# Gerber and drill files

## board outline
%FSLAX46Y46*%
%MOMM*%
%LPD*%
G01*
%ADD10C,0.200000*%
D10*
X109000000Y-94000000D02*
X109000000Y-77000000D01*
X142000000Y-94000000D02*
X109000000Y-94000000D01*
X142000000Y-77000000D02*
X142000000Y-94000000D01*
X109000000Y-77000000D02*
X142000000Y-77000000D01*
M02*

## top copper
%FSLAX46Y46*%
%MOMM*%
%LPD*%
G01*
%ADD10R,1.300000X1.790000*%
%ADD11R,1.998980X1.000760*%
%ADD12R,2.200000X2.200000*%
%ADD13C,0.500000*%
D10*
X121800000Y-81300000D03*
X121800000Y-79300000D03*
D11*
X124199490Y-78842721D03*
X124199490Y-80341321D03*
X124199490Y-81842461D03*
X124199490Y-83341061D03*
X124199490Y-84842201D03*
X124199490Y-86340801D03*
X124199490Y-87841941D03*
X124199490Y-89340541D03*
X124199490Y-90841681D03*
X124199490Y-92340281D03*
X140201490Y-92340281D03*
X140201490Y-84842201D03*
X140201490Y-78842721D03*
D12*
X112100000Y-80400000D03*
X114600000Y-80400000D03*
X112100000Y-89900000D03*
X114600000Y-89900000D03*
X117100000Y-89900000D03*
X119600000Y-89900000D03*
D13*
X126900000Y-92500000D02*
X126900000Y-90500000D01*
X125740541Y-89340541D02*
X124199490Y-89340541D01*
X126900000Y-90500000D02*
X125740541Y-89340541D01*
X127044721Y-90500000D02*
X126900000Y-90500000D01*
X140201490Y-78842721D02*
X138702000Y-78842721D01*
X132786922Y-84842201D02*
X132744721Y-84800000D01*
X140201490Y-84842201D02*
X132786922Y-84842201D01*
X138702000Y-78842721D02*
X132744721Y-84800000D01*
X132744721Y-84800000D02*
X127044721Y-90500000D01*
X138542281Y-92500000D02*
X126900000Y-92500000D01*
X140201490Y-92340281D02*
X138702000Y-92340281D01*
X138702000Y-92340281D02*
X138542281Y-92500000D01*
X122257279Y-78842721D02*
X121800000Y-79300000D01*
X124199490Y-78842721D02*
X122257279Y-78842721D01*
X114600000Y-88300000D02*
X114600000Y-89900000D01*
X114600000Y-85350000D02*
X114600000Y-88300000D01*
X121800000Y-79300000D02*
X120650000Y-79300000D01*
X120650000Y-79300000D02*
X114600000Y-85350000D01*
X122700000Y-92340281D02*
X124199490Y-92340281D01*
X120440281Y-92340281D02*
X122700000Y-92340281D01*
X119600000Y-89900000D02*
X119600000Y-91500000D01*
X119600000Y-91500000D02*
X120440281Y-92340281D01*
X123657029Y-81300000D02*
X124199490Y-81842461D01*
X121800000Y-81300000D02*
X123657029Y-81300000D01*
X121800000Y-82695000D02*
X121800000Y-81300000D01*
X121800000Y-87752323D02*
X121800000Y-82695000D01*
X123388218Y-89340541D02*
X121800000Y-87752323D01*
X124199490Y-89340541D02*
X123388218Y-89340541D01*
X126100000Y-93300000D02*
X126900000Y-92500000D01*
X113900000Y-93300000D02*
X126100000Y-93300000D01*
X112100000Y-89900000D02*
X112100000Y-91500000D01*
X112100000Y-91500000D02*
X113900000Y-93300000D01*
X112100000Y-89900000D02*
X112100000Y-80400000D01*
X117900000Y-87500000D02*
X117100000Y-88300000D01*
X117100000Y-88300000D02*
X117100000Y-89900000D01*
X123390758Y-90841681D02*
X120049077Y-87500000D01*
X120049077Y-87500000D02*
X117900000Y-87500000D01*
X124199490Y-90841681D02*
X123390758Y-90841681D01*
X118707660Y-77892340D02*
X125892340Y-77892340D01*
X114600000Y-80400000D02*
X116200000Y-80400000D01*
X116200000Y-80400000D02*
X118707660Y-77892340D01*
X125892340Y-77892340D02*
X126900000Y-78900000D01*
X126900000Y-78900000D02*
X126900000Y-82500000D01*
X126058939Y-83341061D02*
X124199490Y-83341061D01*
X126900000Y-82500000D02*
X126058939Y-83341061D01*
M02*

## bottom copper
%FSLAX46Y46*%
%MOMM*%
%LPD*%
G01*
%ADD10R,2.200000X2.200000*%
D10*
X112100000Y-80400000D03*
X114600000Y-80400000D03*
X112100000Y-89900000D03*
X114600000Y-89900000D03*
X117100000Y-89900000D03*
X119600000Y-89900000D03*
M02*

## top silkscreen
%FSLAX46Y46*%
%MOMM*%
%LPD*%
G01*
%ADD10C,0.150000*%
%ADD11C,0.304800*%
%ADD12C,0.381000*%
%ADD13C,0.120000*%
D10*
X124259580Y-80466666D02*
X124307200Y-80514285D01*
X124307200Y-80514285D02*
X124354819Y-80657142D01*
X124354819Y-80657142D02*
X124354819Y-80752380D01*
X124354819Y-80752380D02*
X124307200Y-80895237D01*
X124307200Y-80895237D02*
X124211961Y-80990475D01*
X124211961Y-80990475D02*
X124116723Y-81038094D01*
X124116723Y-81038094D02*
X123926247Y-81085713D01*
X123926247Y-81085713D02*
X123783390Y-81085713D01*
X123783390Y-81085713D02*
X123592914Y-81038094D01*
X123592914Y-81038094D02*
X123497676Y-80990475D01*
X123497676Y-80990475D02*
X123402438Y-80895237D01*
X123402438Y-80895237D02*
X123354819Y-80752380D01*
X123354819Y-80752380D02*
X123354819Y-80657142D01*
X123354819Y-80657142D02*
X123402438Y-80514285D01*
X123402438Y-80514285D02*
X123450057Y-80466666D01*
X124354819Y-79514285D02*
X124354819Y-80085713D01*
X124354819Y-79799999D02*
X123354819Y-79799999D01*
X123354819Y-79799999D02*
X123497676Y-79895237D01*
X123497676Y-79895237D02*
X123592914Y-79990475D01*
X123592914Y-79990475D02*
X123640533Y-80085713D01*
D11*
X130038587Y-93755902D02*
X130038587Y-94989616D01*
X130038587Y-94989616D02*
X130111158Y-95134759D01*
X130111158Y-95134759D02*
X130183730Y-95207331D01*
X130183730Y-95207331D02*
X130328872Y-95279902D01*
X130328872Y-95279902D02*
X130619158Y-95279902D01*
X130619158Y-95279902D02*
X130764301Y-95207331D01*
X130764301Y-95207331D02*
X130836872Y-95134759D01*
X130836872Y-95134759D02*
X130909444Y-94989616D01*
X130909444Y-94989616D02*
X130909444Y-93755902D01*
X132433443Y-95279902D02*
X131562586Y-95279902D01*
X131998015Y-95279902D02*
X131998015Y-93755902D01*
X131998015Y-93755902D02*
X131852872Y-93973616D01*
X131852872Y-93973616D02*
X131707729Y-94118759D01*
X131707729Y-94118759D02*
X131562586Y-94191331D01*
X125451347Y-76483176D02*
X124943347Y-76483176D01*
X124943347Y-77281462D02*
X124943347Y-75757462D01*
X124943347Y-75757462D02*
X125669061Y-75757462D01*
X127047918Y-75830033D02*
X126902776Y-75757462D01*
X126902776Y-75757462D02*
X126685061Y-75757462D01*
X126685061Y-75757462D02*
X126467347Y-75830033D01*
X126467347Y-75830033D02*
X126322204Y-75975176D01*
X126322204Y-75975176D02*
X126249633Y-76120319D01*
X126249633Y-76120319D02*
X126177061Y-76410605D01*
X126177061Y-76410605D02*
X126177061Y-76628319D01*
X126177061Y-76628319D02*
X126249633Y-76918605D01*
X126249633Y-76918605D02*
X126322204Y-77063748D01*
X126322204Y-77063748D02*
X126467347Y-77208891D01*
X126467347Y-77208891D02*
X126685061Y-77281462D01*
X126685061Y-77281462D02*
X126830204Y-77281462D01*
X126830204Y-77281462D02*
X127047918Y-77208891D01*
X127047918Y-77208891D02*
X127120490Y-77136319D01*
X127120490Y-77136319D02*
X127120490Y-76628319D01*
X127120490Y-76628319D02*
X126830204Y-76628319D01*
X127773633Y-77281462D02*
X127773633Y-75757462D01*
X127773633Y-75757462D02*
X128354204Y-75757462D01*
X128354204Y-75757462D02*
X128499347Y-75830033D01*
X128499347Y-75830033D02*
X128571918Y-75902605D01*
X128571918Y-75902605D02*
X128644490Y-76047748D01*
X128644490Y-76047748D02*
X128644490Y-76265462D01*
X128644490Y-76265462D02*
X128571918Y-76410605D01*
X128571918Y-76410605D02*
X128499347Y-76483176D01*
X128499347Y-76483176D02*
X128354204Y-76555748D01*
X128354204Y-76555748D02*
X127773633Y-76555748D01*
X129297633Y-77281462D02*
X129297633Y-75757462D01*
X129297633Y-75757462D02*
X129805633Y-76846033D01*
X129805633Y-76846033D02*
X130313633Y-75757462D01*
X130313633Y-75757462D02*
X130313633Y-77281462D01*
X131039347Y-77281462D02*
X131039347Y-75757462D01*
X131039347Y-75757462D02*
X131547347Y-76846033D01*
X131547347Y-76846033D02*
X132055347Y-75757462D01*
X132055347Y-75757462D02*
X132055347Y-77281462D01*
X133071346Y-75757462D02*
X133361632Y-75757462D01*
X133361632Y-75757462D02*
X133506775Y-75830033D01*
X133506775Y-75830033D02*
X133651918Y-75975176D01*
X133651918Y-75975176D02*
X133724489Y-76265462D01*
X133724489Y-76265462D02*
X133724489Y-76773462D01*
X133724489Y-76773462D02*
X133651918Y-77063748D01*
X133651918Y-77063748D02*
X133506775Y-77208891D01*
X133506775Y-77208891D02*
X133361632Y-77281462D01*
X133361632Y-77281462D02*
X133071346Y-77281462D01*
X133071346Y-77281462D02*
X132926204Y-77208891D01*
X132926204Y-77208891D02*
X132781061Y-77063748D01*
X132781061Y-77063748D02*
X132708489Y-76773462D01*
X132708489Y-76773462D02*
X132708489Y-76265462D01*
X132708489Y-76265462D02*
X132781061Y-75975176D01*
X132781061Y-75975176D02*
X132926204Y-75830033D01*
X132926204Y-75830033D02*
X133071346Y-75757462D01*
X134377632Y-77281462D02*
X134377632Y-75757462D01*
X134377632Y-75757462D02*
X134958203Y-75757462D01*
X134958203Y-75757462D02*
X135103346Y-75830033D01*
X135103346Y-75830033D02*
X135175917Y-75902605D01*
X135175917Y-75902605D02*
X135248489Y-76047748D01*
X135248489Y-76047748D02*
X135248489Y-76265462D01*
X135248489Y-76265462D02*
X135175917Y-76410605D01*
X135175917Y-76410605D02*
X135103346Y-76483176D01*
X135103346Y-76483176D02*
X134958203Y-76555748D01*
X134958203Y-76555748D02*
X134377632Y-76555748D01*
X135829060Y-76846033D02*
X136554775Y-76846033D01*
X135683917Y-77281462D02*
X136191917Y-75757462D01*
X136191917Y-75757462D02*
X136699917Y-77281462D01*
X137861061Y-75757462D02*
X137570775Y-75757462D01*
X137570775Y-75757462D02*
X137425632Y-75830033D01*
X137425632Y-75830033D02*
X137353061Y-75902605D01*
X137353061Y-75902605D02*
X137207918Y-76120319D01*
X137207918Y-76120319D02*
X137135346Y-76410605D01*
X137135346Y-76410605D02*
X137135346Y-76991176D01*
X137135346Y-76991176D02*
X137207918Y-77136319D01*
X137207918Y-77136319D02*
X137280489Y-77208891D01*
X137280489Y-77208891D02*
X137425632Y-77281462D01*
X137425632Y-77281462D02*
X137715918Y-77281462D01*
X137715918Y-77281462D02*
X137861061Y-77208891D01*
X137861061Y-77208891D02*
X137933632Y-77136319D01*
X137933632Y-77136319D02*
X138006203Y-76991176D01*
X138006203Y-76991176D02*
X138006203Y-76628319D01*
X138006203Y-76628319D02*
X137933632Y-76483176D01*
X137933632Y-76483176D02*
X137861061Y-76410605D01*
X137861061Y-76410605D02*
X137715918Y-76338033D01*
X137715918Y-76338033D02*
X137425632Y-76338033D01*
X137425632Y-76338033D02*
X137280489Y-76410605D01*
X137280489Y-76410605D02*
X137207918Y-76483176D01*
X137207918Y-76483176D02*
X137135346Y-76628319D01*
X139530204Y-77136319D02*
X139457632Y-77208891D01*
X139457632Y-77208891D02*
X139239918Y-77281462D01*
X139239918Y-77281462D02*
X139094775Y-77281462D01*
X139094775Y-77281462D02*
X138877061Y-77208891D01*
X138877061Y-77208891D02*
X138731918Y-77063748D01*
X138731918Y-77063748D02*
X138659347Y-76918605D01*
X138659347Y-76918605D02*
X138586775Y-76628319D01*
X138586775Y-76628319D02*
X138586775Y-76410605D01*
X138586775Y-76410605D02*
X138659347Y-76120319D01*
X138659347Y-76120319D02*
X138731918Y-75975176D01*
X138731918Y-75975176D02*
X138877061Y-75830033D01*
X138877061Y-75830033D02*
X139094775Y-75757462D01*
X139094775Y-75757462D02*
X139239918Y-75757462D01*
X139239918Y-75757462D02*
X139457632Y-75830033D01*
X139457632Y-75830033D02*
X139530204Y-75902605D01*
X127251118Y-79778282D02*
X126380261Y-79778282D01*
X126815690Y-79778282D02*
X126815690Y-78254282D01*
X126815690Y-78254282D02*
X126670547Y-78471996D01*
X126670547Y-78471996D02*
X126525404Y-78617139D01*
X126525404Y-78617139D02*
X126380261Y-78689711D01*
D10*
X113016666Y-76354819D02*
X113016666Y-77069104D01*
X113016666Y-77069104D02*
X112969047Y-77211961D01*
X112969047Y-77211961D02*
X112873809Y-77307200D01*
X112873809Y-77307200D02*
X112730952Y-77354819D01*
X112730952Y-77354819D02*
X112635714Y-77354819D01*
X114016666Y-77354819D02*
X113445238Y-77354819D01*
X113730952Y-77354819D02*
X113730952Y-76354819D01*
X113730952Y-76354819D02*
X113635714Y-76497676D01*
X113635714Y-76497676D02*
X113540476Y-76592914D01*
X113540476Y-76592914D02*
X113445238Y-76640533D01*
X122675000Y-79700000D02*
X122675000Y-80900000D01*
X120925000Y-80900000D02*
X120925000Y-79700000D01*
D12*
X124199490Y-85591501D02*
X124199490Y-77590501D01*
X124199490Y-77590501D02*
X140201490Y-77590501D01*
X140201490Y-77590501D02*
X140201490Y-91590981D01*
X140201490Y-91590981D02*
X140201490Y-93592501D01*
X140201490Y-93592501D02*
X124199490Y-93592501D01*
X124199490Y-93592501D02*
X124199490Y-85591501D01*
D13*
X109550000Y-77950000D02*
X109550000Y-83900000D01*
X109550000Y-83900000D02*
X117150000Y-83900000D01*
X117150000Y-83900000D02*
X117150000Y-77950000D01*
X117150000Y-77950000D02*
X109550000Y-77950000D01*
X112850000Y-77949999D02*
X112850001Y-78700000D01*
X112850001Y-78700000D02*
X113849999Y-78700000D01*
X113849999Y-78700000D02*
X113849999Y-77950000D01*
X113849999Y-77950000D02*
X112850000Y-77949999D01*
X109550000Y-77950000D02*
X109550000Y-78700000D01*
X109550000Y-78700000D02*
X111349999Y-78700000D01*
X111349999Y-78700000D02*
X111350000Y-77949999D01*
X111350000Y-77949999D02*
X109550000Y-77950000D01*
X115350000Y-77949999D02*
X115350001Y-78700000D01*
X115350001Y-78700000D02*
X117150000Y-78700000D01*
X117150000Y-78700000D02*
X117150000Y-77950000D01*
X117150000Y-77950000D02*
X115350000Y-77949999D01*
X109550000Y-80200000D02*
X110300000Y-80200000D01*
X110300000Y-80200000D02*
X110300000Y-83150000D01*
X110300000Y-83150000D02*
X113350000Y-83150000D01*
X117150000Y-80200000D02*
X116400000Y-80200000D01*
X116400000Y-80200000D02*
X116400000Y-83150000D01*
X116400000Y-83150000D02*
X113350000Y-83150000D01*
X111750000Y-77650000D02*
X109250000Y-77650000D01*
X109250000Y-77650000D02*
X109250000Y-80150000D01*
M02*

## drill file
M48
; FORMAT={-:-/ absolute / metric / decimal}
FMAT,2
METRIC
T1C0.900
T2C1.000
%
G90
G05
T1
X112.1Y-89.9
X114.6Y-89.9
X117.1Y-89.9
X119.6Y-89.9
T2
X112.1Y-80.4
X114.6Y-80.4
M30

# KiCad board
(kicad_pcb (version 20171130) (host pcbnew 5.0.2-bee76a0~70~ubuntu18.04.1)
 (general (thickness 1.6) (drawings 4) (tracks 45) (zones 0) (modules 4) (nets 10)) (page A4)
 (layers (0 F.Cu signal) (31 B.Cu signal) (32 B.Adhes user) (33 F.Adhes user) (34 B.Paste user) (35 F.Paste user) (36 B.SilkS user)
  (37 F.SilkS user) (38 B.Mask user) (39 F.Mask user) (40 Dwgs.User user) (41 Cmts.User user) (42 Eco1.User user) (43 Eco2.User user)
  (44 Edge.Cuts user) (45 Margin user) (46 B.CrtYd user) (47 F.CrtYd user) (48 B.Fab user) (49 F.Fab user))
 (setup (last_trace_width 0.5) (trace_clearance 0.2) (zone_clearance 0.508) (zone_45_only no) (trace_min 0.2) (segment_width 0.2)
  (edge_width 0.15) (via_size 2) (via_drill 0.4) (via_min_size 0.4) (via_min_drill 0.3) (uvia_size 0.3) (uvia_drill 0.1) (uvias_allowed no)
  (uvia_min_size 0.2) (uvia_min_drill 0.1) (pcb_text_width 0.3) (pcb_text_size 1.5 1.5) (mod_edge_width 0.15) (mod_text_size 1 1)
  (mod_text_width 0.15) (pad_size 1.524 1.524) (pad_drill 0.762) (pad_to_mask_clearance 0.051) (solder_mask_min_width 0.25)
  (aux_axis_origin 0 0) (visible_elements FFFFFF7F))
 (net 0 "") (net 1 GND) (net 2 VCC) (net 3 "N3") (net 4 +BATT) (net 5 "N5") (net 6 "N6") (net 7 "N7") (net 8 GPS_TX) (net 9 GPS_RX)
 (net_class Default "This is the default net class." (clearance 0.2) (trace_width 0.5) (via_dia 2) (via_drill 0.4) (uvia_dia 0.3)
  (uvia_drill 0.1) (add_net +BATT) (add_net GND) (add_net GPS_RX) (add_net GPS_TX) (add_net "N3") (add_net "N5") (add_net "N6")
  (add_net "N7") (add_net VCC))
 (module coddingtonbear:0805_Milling (layer F.Cu) (at 121.8 80.3 270)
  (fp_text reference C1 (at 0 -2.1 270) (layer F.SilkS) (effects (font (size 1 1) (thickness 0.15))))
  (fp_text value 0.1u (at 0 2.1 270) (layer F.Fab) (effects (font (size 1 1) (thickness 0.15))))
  (fp_line (start -0.6 -0.875) (end 0.6 -0.875) (layer F.SilkS) (width 0.15))
  (fp_line (start 0.6 0.875) (end -0.6 0.875) (layer F.SilkS) (width 0.15))
  (pad 2 smd rect (at 1 0 270) (size 1.79 1.3) (layers F.Cu F.Paste F.Mask) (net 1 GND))
  (pad 1 smd rect (at -1 0 270) (size 1.79 1.3) (layers F.Cu F.Paste F.Mask) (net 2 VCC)))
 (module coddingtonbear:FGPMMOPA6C (layer F.Cu) (at 132.20049 85.591501)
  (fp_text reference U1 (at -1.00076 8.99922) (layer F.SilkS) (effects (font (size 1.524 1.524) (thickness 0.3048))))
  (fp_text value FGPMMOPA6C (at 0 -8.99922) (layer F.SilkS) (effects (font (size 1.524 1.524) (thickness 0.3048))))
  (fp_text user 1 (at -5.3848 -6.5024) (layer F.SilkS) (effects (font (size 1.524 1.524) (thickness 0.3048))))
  (fp_line (start -8.001 0) (end -8.001 -8.001) (layer F.SilkS) (width 0.381))
  (fp_line (start -8.001 -8.001) (end 8.001 -8.001) (layer F.SilkS) (width 0.381))
  (fp_line (start 8.001 -8.001) (end 8.001 5.99948) (layer F.SilkS) (width 0.381))
  (fp_line (start 8.001 5.99948) (end 8.001 8.001) (layer F.SilkS) (width 0.381))
  (fp_line (start 8.001 8.001) (end -8.001 8.001) (layer F.SilkS) (width 0.381))
  (fp_line (start -8.001 8.001) (end -8.001 0) (layer F.SilkS) (width 0.381))
  (pad 1 smd rect (at -8.001 -6.74878) (size 1.99898 1.00076) (layers F.Cu F.Paste F.Mask) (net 2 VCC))
  (pad 2 smd rect (at -8.001 -5.25018) (size 1.99898 1.00076) (layers F.Cu F.Paste F.Mask) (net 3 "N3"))
  (pad 3 smd rect (at -8.001 -3.74904) (size 1.99898 1.00076) (layers F.Cu F.Paste F.Mask) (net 1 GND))
  (pad 4 smd rect (at -8.001 -2.25044) (size 1.99898 1.00076) (layers F.Cu F.Paste F.Mask) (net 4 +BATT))
  (pad 5 smd rect (at -8.001 -0.7493) (size 1.99898 1.00076) (layers F.Cu F.Paste F.Mask) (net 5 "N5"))
  (pad 6 smd rect (at -8.001 0.7493) (size 1.99898 1.00076) (layers F.Cu F.Paste F.Mask) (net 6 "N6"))
  (pad 7 smd rect (at -8.001 2.25044) (size 1.99898 1.00076) (layers F.Cu F.Paste F.Mask) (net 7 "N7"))
  (pad 8 smd rect (at -8.001 3.74904) (size 1.99898 1.00076) (layers F.Cu F.Paste F.Mask) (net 1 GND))
  (pad 9 smd rect (at -8.001 5.25018) (size 1.99898 1.00076) (layers F.Cu F.Paste F.Mask) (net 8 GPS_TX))
  (pad 10 smd rect (at -8.001 6.74878) (size 1.99898 1.00076) (layers F.Cu F.Paste F.Mask) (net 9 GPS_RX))
  (pad 11 smd rect (at 8.001 6.74878) (size 1.99898 1.00076) (layers F.Cu F.Paste F.Mask) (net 1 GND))
  (pad 12 smd rect (at 8.001 -0.7493) (size 1.99898 1.00076) (layers F.Cu F.Paste F.Mask) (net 1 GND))
  (pad 13 smd rect (at 8.001 -6.74878) (size 1.99898 1.00076) (layers F.Cu F.Paste F.Mask) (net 1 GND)))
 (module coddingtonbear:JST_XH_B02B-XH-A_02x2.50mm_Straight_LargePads (layer F.Cu) (at 112.1 80.4)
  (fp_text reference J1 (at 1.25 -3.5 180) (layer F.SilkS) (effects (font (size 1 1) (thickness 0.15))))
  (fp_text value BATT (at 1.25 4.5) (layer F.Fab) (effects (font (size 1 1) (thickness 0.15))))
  (fp_line (start -2.55 -2.45) (end -2.55 3.5) (layer F.SilkS) (width 0.12))
  (fp_line (start -2.55 3.5) (end 5.05 3.5) (layer F.SilkS) (width 0.12))
  (fp_line (start 5.05 3.5) (end 5.05 -2.45) (layer F.SilkS) (width 0.12))
  (fp_line (start 5.05 -2.45) (end -2.55 -2.45) (layer F.SilkS) (width 0.12))
  (fp_line (start 0.75 -2.450001) (end 0.750001 -1.7) (layer F.SilkS) (width 0.12))
  (fp_line (start 0.750001 -1.7) (end 1.749999 -1.7) (layer F.SilkS) (width 0.12))
  (fp_line (start 1.749999 -1.7) (end 1.749999 -2.45) (layer F.SilkS) (width 0.12))
  (fp_line (start 1.749999 -2.45) (end 0.75 -2.450001) (layer F.SilkS) (width 0.12))
  (fp_line (start -2.55 -2.45) (end -2.55 -1.7) (layer F.SilkS) (width 0.12))
  (fp_line (start -2.55 -1.7) (end -0.750001 -1.7) (layer F.SilkS) (width 0.12))
  (fp_line (start -0.750001 -1.7) (end -0.75 -2.450001) (layer F.SilkS) (width 0.12))
  (fp_line (start -0.75 -2.450001) (end -2.55 -2.45) (layer F.SilkS) (width 0.12))
  (fp_line (start 3.25 -2.450001) (end 3.250001 -1.7) (layer F.SilkS) (width 0.12))
  (fp_line (start 3.250001 -1.7) (end 5.05 -1.7) (layer F.SilkS) (width 0.12))
  (fp_line (start 5.05 -1.7) (end 5.05 -2.45) (layer F.SilkS) (width 0.12))
  (fp_line (start 5.05 -2.45) (end 3.25 -2.450001) (layer F.SilkS) (width 0.12))
  (fp_line (start -2.55 -0.2) (end -1.8 -0.2) (layer F.SilkS) (width 0.12))
  (fp_line (start -1.8 -0.2) (end -1.8 2.75) (layer F.SilkS) (width 0.12))
  (fp_line (start -1.8 2.75) (end 1.25 2.75) (layer F.SilkS) (width 0.12))
  (fp_line (start 5.05 -0.2) (end 4.3 -0.2) (layer F.SilkS) (width 0.12))
  (fp_line (start 4.3 -0.2) (end 4.3 2.75) (layer F.SilkS) (width 0.12))
  (fp_line (start 4.3 2.75) (end 1.25 2.75) (layer F.SilkS) (width 0.12))
  (fp_line (start -0.35 -2.75) (end -2.85 -2.75) (layer F.SilkS) (width 0.12))
  (fp_line (start -2.85 -2.75) (end -2.85 -0.25) (layer F.SilkS) (width 0.12))
  (pad 1 thru_hole rect (at 0 0) (size 2.2 2.2) (drill 1) (layers *.Cu *.Mask) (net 1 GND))
  (pad 2 thru_hole rect (at 2.5 0) (size 2.2 2.2) (drill 1) (layers *.Cu *.Mask) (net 4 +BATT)))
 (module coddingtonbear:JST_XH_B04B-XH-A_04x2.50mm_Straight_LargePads (layer B.Cu) (at 112.1 89.9)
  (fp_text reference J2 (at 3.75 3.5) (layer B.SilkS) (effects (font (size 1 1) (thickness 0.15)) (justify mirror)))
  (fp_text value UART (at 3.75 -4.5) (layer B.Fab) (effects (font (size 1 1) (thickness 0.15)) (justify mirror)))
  (pad 1 thru_hole rect (at 0 0) (size 2.2 2.2) (drill 0.9) (layers *.Cu *.Mask) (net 1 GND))
  (pad 2 thru_hole rect (at 2.5 0) (size 2.2 2.2) (drill 0.9) (layers *.Cu *.Mask) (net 2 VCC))
  (pad 3 thru_hole rect (at 5 0) (size 2.2 2.2) (drill 0.9) (layers *.Cu *.Mask) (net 8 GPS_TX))
  (pad 4 thru_hole rect (at 7.5 0) (size 2.2 2.2) (drill 0.9) (layers *.Cu *.Mask) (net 9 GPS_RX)))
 (gr_line (start 109 94) (end 109 77) (layer Edge.Cuts) (width 0.2))
 (gr_line (start 142 94) (end 109 94) (layer Edge.Cuts) (width 0.2))
 (gr_line (start 142 77) (end 142 94) (layer Edge.Cuts) (width 0.2))
 (gr_line (start 109 77) (end 142 77) (layer Edge.Cuts) (width 0.2))
 (segment (start 126.9 92.5) (end 126.9 90.5) (width 0.5) (layer F.Cu) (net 1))
 (segment (start 125.740541 89.340541) (end 124.19949 89.340541) (width 0.5) (layer F.Cu) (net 1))
 (segment (start 126.9 90.5) (end 125.740541 89.340541) (width 0.5) (layer F.Cu) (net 1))
 (segment (start 127.044721 90.5) (end 126.9 90.5) (width 0.5) (layer F.Cu) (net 1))
 (segment (start 140.20149 78.842721) (end 138.702 78.842721) (width 0.5) (layer F.Cu) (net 1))
 (segment (start 132.786922 84.842201) (end 132.744721 84.8) (width 0.5) (layer F.Cu) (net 1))
 (segment (start 140.20149 84.842201) (end 132.786922 84.842201) (width 0.5) (layer F.Cu) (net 1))
 (segment (start 138.702 78.842721) (end 132.744721 84.8) (width 0.5) (layer F.Cu) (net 1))
 (segment (start 132.744721 84.8) (end 127.044721 90.5) (width 0.5) (layer F.Cu) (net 1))
 (segment (start 138.542281 92.5) (end 126.9 92.5) (width 0.5) (layer F.Cu) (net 1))
 (segment (start 140.20149 92.340281) (end 138.702 92.340281) (width 0.5) (layer F.Cu) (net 1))
 (segment (start 138.702 92.340281) (end 138.542281 92.5) (width 0.5) (layer F.Cu) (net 1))
 (segment (start 122.257279 78.842721) (end 121.8 79.3) (width 0.5) (layer F.Cu) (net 2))
 (segment (start 124.19949 78.842721) (end 122.257279 78.842721) (width 0.5) (layer F.Cu) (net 2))
 (segment (start 114.6 88.3) (end 114.6 89.9) (width 0.5) (layer F.Cu) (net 2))
 (segment (start 114.6 85.35) (end 114.6 88.3) (width 0.5) (layer F.Cu) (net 2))
 (segment (start 121.8 79.3) (end 120.65 79.3) (width 0.5) (layer F.Cu) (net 2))
 (segment (start 120.65 79.3) (end 114.6 85.35) (width 0.5) (layer F.Cu) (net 2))
 (segment (start 122.7 92.340281) (end 124.19949 92.340281) (width 0.5) (layer F.Cu) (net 9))
 (segment (start 120.440281 92.340281) (end 122.7 92.340281) (width 0.5) (layer F.Cu) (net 9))
 (segment (start 119.6 89.9) (end 119.6 91.5) (width 0.5) (layer F.Cu) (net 9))
 (segment (start 119.6 91.5) (end 120.440281 92.340281) (width 0.5) (layer F.Cu) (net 9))
 (segment (start 123.657029 81.3) (end 124.19949 81.842461) (width 0.5) (layer F.Cu) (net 1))
 (segment (start 121.8 81.3) (end 123.657029 81.3) (width 0.5) (layer F.Cu) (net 1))
 (segment (start 121.8 82.695) (end 121.8 81.3) (width 0.5) (layer F.Cu) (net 1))
 (segment (start 121.8 87.752323) (end 121.8 82.695) (width 0.5) (layer F.Cu) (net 1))
 (segment (start 123.388218 89.340541) (end 121.8 87.752323) (width 0.5) (layer F.Cu) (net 1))
 (segment (start 124.19949 89.340541) (end 123.388218 89.340541) (width 0.5) (layer F.Cu) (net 1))
 (segment (start 126.1 93.3) (end 126.9 92.5) (width 0.5) (layer F.Cu) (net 1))
 (segment (start 113.9 93.3) (end 126.1 93.3) (width 0.5) (layer F.Cu) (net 1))
 (segment (start 112.1 89.9) (end 112.1 91.5) (width 0.5) (layer F.Cu) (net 1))
 (segment (start 112.1 91.5) (end 113.9 93.3) (width 0.5) (layer F.Cu) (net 1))
 (segment (start 112.1 89.9) (end 112.1 80.4) (width 0.5) (layer F.Cu) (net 1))
 (segment (start 117.9 87.5) (end 117.1 88.3) (width 0.5) (layer F.Cu) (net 8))
 (segment (start 117.1 88.3) (end 117.1 89.9) (width 0.5) (layer F.Cu) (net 8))
 (segment (start 123.390758 90.841681) (end 120.049077 87.5) (width 0.5) (layer F.Cu) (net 8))
 (segment (start 120.049077 87.5) (end 117.9 87.5) (width 0.5) (layer F.Cu) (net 8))
 (segment (start 124.19949 90.841681) (end 123.390758 90.841681) (width 0.5) (layer F.Cu) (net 8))
 (segment (start 118.70766 77.89234) (end 125.89234 77.89234) (width 0.5) (layer F.Cu) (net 4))
 (segment (start 114.6 80.4) (end 116.2 80.4) (width 0.5) (layer F.Cu) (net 4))
 (segment (start 116.2 80.4) (end 118.70766 77.89234) (width 0.5) (layer F.Cu) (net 4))
 (segment (start 125.89234 77.89234) (end 126.9 78.9) (width 0.5) (layer F.Cu) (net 4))
 (segment (start 126.9 78.9) (end 126.9 82.5) (width 0.5) (layer F.Cu) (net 4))
 (segment (start 126.058939 83.341061) (end 124.19949 83.341061) (width 0.5) (layer F.Cu) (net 4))
 (segment (start 126.9 82.5) (end 126.058939 83.341061) (width 0.5) (layer F.Cu) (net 4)))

